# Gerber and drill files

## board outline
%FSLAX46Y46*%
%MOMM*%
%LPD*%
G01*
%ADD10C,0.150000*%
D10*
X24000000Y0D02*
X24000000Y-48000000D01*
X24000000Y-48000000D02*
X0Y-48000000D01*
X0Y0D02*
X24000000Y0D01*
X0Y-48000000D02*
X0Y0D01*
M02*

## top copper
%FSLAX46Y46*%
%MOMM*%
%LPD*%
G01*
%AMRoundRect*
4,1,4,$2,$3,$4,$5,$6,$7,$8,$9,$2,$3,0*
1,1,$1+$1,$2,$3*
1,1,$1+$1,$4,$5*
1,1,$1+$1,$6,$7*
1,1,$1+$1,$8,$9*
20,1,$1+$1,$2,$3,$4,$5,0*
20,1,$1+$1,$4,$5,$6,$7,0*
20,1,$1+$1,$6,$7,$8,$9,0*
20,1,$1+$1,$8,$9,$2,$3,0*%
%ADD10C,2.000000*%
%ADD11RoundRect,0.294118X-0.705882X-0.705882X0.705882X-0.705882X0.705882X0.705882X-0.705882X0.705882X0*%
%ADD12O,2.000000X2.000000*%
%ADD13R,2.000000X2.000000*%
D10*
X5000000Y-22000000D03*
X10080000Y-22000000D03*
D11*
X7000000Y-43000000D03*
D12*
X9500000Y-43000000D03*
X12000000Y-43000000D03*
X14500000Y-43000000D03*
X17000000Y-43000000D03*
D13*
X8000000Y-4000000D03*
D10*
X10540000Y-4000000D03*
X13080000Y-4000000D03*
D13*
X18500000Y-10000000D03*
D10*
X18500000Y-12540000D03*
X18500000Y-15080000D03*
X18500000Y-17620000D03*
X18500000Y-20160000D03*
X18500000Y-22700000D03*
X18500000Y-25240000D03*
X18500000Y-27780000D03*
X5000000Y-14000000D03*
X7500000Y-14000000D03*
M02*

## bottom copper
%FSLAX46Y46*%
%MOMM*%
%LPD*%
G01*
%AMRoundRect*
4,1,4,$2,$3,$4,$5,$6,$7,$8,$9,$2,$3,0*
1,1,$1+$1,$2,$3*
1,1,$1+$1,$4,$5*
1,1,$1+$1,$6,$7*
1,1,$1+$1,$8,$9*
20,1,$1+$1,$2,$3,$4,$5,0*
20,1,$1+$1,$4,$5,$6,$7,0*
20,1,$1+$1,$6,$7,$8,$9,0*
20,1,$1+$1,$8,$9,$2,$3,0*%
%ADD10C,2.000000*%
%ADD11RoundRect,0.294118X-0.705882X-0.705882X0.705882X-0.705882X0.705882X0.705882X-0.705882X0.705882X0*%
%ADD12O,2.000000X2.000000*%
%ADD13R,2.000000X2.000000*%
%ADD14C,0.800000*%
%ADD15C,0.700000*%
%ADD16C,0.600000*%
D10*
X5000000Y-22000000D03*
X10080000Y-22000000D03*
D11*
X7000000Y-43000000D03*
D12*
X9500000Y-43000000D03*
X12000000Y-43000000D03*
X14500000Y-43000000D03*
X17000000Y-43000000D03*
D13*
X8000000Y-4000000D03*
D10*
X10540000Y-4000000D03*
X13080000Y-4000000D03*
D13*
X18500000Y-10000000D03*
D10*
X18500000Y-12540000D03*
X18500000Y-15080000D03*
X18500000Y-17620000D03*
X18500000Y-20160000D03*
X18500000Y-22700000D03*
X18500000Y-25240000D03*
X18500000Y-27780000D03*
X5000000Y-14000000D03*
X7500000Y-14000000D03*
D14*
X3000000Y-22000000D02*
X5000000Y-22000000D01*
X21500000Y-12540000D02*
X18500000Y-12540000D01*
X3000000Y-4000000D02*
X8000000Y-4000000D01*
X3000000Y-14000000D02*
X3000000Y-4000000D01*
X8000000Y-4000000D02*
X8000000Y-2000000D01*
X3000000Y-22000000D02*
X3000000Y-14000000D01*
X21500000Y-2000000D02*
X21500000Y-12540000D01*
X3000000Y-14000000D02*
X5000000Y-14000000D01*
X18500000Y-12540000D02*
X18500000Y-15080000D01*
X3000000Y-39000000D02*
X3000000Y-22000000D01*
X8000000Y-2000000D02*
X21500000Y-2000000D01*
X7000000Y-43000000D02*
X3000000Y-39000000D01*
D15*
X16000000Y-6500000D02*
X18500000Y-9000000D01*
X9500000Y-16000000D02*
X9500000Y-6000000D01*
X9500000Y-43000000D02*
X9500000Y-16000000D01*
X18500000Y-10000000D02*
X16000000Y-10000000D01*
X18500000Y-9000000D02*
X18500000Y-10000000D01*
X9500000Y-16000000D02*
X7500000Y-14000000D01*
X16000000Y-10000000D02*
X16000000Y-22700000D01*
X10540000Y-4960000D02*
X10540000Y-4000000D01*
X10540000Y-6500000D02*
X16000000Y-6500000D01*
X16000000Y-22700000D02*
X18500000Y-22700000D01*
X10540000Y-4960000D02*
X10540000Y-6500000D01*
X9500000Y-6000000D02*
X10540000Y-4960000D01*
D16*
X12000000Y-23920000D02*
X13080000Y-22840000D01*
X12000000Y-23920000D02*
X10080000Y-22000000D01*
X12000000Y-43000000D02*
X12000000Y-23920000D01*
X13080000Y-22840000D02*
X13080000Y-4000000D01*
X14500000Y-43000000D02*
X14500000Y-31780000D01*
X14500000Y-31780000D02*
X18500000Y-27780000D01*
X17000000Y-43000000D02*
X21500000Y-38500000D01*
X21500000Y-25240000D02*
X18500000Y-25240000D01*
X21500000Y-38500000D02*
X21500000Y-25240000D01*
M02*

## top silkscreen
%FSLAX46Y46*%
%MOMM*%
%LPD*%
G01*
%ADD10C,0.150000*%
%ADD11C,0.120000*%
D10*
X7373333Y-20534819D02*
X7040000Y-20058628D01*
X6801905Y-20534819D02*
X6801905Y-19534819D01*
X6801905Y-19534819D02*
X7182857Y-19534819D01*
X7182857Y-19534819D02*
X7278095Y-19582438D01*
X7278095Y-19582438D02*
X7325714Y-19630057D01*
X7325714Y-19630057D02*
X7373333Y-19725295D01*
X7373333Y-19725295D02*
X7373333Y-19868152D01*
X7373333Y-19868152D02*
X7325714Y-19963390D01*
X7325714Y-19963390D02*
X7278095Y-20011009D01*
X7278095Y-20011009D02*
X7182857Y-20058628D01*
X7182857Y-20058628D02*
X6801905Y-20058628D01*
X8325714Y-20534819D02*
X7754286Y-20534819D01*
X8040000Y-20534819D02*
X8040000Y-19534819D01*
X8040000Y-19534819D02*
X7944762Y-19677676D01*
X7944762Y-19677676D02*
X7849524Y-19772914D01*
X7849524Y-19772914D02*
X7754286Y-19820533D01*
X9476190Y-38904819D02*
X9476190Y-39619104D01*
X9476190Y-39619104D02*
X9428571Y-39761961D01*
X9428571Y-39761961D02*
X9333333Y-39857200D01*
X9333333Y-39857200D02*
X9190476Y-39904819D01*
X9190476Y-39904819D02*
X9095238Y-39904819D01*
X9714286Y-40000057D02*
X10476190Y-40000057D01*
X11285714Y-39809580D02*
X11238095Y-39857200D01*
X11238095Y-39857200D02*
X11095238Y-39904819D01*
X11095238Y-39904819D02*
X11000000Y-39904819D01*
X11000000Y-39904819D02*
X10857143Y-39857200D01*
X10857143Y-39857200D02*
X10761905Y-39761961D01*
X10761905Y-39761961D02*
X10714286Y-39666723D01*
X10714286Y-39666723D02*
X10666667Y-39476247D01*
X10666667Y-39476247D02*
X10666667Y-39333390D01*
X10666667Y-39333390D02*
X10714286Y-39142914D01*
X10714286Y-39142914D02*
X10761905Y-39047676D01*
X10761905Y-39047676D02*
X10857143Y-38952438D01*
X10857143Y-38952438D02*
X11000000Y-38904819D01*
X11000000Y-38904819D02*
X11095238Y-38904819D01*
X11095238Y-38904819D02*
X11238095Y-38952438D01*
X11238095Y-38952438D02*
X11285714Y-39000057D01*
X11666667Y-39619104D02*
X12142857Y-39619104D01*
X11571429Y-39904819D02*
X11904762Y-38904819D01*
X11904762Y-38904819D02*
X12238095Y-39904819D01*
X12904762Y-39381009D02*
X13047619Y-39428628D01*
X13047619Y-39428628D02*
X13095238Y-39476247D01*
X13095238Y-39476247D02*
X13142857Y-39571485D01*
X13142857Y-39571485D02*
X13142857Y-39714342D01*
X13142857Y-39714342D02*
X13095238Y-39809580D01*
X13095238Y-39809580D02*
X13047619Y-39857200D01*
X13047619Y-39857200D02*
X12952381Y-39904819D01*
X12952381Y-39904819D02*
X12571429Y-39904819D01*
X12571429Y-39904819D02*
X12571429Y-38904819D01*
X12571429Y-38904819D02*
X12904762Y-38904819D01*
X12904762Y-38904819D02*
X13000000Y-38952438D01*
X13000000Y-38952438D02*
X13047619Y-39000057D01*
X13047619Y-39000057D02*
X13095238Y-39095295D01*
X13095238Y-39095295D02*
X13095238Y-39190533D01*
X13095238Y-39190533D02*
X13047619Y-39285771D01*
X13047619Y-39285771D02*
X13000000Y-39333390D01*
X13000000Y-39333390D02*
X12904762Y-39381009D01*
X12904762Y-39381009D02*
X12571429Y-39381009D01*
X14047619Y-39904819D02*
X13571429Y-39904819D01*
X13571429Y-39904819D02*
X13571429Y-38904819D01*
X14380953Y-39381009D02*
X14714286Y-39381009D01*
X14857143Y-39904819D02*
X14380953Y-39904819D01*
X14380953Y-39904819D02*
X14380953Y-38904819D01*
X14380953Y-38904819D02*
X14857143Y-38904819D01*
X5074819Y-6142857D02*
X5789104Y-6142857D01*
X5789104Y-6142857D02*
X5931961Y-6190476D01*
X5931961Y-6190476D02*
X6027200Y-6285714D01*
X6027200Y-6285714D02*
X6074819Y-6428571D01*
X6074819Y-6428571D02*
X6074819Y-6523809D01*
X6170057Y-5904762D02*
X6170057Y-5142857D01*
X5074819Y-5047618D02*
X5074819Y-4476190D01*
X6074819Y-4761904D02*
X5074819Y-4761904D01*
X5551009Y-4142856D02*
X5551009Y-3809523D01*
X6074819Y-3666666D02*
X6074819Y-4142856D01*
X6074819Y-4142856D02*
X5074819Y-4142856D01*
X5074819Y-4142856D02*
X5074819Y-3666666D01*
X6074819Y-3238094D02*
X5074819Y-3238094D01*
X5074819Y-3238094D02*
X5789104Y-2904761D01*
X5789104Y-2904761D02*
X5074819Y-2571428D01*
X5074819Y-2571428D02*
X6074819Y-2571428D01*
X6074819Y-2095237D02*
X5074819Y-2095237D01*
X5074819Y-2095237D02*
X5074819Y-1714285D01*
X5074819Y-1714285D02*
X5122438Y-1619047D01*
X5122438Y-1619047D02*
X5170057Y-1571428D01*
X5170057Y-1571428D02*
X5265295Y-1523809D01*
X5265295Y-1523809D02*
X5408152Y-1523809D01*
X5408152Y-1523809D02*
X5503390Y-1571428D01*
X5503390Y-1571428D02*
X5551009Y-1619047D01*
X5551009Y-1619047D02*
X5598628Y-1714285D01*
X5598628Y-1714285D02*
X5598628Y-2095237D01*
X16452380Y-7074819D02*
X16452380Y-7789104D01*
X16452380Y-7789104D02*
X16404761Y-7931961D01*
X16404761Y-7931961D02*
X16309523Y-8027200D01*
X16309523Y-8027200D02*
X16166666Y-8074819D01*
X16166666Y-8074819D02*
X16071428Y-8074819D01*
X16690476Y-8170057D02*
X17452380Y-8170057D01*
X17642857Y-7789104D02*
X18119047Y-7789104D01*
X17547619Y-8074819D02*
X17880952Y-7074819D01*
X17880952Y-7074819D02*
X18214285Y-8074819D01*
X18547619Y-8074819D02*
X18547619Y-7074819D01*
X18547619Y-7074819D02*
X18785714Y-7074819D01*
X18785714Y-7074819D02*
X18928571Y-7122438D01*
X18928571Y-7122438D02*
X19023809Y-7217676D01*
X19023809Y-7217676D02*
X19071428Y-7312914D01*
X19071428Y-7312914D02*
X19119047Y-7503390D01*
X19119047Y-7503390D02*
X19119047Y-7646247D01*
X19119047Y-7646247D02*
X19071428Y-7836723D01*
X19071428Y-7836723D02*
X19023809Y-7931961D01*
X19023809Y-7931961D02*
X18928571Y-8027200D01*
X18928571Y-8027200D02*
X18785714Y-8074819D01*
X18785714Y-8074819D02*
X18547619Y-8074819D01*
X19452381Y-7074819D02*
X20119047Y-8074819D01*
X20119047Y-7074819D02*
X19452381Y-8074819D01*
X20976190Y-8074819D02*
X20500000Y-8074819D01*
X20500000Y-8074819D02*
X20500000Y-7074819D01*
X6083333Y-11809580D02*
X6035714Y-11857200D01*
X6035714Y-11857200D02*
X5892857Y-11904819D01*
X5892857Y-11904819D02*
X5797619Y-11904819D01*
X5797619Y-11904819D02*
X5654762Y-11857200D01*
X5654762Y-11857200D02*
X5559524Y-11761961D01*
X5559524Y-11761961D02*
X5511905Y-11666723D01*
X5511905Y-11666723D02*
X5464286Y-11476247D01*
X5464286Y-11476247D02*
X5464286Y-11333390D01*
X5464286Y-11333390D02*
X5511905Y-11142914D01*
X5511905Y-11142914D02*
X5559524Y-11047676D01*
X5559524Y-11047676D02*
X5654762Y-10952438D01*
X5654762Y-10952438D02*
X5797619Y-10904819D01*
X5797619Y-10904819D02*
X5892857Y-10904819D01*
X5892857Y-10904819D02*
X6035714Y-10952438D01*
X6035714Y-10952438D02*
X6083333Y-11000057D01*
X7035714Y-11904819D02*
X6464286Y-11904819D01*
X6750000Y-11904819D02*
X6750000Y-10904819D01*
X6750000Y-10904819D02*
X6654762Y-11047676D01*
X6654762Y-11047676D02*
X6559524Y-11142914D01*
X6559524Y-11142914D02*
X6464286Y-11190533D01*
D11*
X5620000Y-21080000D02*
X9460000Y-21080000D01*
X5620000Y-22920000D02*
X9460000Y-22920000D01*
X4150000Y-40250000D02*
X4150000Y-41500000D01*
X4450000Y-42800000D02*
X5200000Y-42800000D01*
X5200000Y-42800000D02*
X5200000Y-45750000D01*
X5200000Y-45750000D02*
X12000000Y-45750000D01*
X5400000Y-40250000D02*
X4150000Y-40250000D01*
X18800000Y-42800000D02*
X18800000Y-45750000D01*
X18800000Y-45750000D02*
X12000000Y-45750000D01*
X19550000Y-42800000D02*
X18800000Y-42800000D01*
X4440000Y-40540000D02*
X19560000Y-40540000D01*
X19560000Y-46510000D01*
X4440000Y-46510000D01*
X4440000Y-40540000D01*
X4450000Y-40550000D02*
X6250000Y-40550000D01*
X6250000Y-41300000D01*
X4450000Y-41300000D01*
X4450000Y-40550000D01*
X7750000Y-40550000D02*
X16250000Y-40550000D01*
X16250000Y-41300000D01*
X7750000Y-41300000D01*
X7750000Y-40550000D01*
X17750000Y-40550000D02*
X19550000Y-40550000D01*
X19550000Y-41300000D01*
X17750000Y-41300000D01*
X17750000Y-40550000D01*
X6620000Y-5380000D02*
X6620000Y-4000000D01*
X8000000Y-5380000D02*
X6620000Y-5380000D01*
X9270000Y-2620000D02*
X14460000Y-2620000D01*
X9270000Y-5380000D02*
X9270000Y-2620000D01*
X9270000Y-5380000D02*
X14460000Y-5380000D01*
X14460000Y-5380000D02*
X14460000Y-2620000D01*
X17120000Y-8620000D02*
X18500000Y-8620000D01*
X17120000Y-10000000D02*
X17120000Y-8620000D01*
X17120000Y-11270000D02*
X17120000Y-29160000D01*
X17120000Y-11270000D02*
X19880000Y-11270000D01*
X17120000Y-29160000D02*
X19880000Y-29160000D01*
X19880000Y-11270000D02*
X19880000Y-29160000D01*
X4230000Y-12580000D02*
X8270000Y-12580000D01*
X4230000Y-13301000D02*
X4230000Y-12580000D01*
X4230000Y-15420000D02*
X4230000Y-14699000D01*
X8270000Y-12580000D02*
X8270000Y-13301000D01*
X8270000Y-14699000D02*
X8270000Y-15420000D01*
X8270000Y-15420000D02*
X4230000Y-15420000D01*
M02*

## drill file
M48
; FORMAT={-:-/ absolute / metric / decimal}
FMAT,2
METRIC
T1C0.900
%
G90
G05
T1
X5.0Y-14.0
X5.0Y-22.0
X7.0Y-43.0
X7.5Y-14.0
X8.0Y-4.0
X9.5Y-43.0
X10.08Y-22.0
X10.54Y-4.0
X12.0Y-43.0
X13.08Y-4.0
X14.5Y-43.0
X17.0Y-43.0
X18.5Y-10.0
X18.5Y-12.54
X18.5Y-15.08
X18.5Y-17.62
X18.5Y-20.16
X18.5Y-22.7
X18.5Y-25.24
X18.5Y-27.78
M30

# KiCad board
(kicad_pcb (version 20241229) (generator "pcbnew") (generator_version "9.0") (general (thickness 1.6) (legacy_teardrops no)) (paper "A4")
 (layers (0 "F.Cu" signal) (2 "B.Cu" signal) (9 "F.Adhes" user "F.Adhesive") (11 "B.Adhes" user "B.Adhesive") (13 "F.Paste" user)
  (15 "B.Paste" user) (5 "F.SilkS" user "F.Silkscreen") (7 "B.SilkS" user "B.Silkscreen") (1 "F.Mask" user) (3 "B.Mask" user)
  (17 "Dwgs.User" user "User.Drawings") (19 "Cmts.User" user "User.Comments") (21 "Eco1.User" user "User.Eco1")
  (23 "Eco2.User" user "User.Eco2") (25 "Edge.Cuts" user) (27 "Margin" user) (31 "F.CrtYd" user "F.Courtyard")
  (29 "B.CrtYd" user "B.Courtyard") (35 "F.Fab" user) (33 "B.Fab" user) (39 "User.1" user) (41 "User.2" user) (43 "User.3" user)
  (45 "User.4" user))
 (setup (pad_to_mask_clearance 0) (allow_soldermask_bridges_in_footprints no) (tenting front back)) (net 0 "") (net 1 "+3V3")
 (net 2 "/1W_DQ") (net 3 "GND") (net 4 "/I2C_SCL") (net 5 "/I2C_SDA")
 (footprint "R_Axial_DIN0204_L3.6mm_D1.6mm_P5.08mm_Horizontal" (layer "F.Cu") (at 5 22)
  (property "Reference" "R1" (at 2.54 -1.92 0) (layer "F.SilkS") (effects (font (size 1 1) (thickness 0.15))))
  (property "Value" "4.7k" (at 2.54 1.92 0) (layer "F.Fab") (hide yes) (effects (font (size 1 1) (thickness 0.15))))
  (fp_line (start 0.62 -0.92) (end 4.46 -0.92) (stroke (width 0.12) (type solid)) (layer "F.SilkS"))
  (fp_line (start 0.62 0.92) (end 4.46 0.92) (stroke (width 0.12) (type solid)) (layer "F.SilkS"))
  (pad "1" thru_hole circle (at 0 0) (size 2 2) (drill 0.9) (layers "*.Cu" "*.Mask") (remove_unused_layers no) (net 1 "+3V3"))
  (pad "2" thru_hole circle (at 5.08 0) (size 2 2) (drill 0.9) (layers "*.Cu" "*.Mask") (remove_unused_layers no) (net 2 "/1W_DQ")))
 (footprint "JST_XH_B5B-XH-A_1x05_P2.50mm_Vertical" (layer "F.Cu") (at 7 43)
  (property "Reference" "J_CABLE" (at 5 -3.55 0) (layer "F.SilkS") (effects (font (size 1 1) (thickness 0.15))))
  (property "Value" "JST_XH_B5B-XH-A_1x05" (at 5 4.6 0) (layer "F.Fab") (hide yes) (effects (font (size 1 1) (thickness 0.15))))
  (fp_line (start -2.85 -2.75) (end -2.85 -1.5) (stroke (width 0.12) (type solid)) (layer "F.SilkS"))
  (fp_line (start -2.55 -0.2) (end -1.8 -0.2) (stroke (width 0.12) (type solid)) (layer "F.SilkS"))
  (fp_line (start -1.8 -0.2) (end -1.8 2.75) (stroke (width 0.12) (type solid)) (layer "F.SilkS"))
  (fp_line (start -1.8 2.75) (end 5 2.75) (stroke (width 0.12) (type solid)) (layer "F.SilkS"))
  (fp_line (start -1.6 -2.75) (end -2.85 -2.75) (stroke (width 0.12) (type solid)) (layer "F.SilkS"))
  (fp_line (start 11.8 -0.2) (end 11.8 2.75) (stroke (width 0.12) (type solid)) (layer "F.SilkS"))
  (fp_line (start 11.8 2.75) (end 5 2.75) (stroke (width 0.12) (type solid)) (layer "F.SilkS"))
  (fp_line (start 12.55 -0.2) (end 11.8 -0.2) (stroke (width 0.12) (type solid)) (layer "F.SilkS"))
  (fp_rect (start -2.56 -2.46) (end 12.56 3.51) (stroke (width 0.12) (type solid)) (fill no) (layer "F.SilkS"))
  (fp_rect (start -2.55 -2.45) (end -0.75 -1.7) (stroke (width 0.12) (type solid)) (fill no) (layer "F.SilkS"))
  (fp_rect (start 0.75 -2.45) (end 9.25 -1.7) (stroke (width 0.12) (type solid)) (fill no) (layer "F.SilkS"))
  (fp_rect (start 10.75 -2.45) (end 12.55 -1.7) (stroke (width 0.12) (type solid)) (fill no) (layer "F.SilkS"))
  (pad "1" thru_hole roundrect (at 0 0) (size 2 2) (drill 0.9) (layers "*.Cu" "*.Mask") (remove_unused_layers no)
   (roundrect_rratio 0.147059) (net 1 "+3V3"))
  (pad "2" thru_hole oval (at 2.5 0) (size 2 2) (drill 0.9) (layers "*.Cu" "*.Mask") (remove_unused_layers no) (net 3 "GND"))
  (pad "3" thru_hole oval (at 5 0) (size 2 2) (drill 0.9) (layers "*.Cu" "*.Mask") (remove_unused_layers no) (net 2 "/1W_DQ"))
  (pad "4" thru_hole oval (at 7.5 0) (size 2 2) (drill 0.9) (layers "*.Cu" "*.Mask") (remove_unused_layers no) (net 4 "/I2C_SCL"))
  (pad "5" thru_hole oval (at 10 0) (size 2 2) (drill 0.9) (layers "*.Cu" "*.Mask") (remove_unused_layers no) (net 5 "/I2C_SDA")))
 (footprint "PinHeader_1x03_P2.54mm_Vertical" (layer "F.Cu") (at 8 4 90)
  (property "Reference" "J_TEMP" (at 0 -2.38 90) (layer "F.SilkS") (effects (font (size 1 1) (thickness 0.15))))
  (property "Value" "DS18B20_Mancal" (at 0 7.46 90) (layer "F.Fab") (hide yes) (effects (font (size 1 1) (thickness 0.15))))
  (fp_line (start -1.38 -1.38) (end 0 -1.38) (stroke (width 0.12) (type solid)) (layer "F.SilkS"))
  (fp_line (start -1.38 0) (end -1.38 -1.38) (stroke (width 0.12) (type solid)) (layer "F.SilkS"))
  (fp_line (start 1.38 1.27) (end 1.38 6.46) (stroke (width 0.12) (type solid)) (layer "F.SilkS"))
  (fp_line (start -1.38 1.27) (end 1.38 1.27) (stroke (width 0.12) (type solid)) (layer "F.SilkS"))
  (fp_line (start -1.38 1.27) (end -1.38 6.46) (stroke (width 0.12) (type solid)) (layer "F.SilkS"))
  (fp_line (start -1.38 6.46) (end 1.38 6.46) (stroke (width 0.12) (type solid)) (layer "F.SilkS"))
  (pad "1" thru_hole rect (at 0 0 90) (size 2 2) (drill 0.9) (layers "*.Cu" "*.Mask") (remove_unused_layers no) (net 1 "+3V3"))
  (pad "2" thru_hole circle (at 0 2.54 90) (size 2 2) (drill 0.9) (layers "*.Cu" "*.Mask") (remove_unused_layers no) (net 3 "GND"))
  (pad "3" thru_hole circle (at 0 5.08 90) (size 2 2) (drill 0.9) (layers "*.Cu" "*.Mask") (remove_unused_layers no) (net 2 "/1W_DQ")))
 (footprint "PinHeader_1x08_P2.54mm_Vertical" (layer "F.Cu") (at 18.5 10)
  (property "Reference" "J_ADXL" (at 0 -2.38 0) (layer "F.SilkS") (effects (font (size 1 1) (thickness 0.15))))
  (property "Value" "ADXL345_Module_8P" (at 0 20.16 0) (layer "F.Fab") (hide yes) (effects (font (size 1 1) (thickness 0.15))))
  (fp_line (start -1.38 -1.38) (end 0 -1.38) (stroke (width 0.12) (type solid)) (layer "F.SilkS"))
  (fp_line (start -1.38 0) (end -1.38 -1.38) (stroke (width 0.12) (type solid)) (layer "F.SilkS"))
  (fp_line (start -1.38 1.27) (end -1.38 19.16) (stroke (width 0.12) (type solid)) (layer "F.SilkS"))
  (fp_line (start -1.38 1.27) (end 1.38 1.27) (stroke (width 0.12) (type solid)) (layer "F.SilkS"))
  (fp_line (start -1.38 19.16) (end 1.38 19.16) (stroke (width 0.12) (type solid)) (layer "F.SilkS"))
  (fp_line (start 1.38 1.27) (end 1.38 19.16) (stroke (width 0.12) (type solid)) (layer "F.SilkS"))
  (pad "1" thru_hole rect (at 0 0) (size 2 2) (drill 0.9) (layers "*.Cu" "*.Mask") (remove_unused_layers no) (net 3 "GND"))
  (pad "2" thru_hole circle (at 0 2.54) (size 2 2) (drill 0.9) (layers "*.Cu" "*.Mask") (remove_unused_layers no) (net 1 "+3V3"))
  (pad "3" thru_hole circle (at 0 5.08) (size 2 2) (drill 0.9) (layers "*.Cu" "*.Mask") (remove_unused_layers no) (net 1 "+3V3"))
  (pad "4" thru_hole circle (at 0 7.62) (size 2 2) (drill 0.9) (layers "*.Cu" "*.Mask") (remove_unused_layers no))
  (pad "5" thru_hole circle (at 0 10.16) (size 2 2) (drill 0.9) (layers "*.Cu" "*.Mask") (remove_unused_layers no))
  (pad "6" thru_hole circle (at 0 12.7) (size 2 2) (drill 0.9) (layers "*.Cu" "*.Mask") (remove_unused_layers no) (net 3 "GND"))
  (pad "7" thru_hole circle (at 0 15.24) (size 2 2) (drill 0.9) (layers "*.Cu" "*.Mask") (remove_unused_layers no) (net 5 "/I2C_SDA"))
  (pad "8" thru_hole circle (at 0 17.78) (size 2 2) (drill 0.9) (layers "*.Cu" "*.Mask") (remove_unused_layers no) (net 4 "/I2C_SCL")))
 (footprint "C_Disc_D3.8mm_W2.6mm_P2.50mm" (layer "F.Cu") (at 5 14)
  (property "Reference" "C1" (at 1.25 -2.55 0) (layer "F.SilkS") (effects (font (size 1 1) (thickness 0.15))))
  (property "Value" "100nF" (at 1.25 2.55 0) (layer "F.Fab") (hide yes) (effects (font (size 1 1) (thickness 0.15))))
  (fp_line (start -0.77 -1.42) (end 3.27 -1.42) (stroke (width 0.12) (type solid)) (layer "F.SilkS"))
  (fp_line (start -0.77 -0.699) (end -0.77 -1.42) (stroke (width 0.12) (type solid)) (layer "F.SilkS"))
  (fp_line (start -0.77 1.42) (end -0.77 0.699) (stroke (width 0.12) (type solid)) (layer "F.SilkS"))
  (fp_line (start 3.27 -1.42) (end 3.27 -0.699) (stroke (width 0.12) (type solid)) (layer "F.SilkS"))
  (fp_line (start 3.27 0.699) (end 3.27 1.42) (stroke (width 0.12) (type solid)) (layer "F.SilkS"))
  (fp_line (start 3.27 1.42) (end -0.77 1.42) (stroke (width 0.12) (type solid)) (layer "F.SilkS"))
  (pad "1" thru_hole circle (at 0 0) (size 2 2) (drill 0.9) (layers "*.Cu" "*.Mask") (remove_unused_layers no) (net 1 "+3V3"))
  (pad "2" thru_hole circle (at 2.5 0) (size 2 2) (drill 0.9) (layers "*.Cu" "*.Mask") (remove_unused_layers no) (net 3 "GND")))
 (gr_line (start 24 0) (end 24 48) (stroke (width 0.15) (type default)) (layer "Edge.Cuts"))
 (gr_line (start 24 48) (end 0 48) (stroke (width 0.15) (type default)) (layer "Edge.Cuts"))
 (gr_line (start 0 0) (end 24 0) (stroke (width 0.15) (type default)) (layer "Edge.Cuts"))
 (gr_line (start 0 48) (end 0 0) (stroke (width 0.15) (type default)) (layer "Edge.Cuts"))
 (segment (start 3 22) (end 5 22) (width 0.8) (layer "B.Cu") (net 1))
 (segment (start 21.5 12.54) (end 18.5 12.54) (width 0.8) (layer "B.Cu") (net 1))
 (segment (start 3 4) (end 8 4) (width 0.8) (layer "B.Cu") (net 1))
 (segment (start 3 14) (end 3 4) (width 0.8) (layer "B.Cu") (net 1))
 (segment (start 8 4) (end 8 2) (width 0.8) (layer "B.Cu") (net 1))
 (segment (start 3 22) (end 3 14) (width 0.8) (layer "B.Cu") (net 1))
 (segment (start 21.5 2) (end 21.5 12.54) (width 0.8) (layer "B.Cu") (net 1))
 (segment (start 3 14) (end 5 14) (width 0.8) (layer "B.Cu") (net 1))
 (segment (start 18.5 12.54) (end 18.5 15.08) (width 0.8) (layer "B.Cu") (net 1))
 (segment (start 3 39) (end 3 22) (width 0.8) (layer "B.Cu") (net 1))
 (segment (start 8 2) (end 21.5 2) (width 0.8) (layer "B.Cu") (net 1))
 (segment (start 7 43) (end 3 39) (width 0.8) (layer "B.Cu") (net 1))
 (segment (start 16 6.5) (end 18.5 9) (width 0.7) (layer "B.Cu") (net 3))
 (segment (start 9.5 16) (end 9.5 6) (width 0.7) (layer "B.Cu") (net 3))
 (segment (start 9.5 43) (end 9.5 16) (width 0.7) (layer "B.Cu") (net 3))
 (segment (start 18.5 10) (end 16 10) (width 0.7) (layer "B.Cu") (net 3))
 (segment (start 18.5 9) (end 18.5 10) (width 0.7) (layer "B.Cu") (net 3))
 (segment (start 9.5 16) (end 7.5 14) (width 0.7) (layer "B.Cu") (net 3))
 (segment (start 16 10) (end 16 22.7) (width 0.7) (layer "B.Cu") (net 3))
 (segment (start 10.54 4.96) (end 10.54 4) (width 0.7) (layer "B.Cu") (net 3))
 (segment (start 10.54 6.5) (end 16 6.5) (width 0.7) (layer "B.Cu") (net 3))
 (segment (start 16 22.7) (end 18.5 22.7) (width 0.7) (layer "B.Cu") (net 3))
 (segment (start 10.54 4.96) (end 10.54 6.5) (width 0.7) (layer "B.Cu") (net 3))
 (segment (start 9.5 6) (end 10.54 4.96) (width 0.7) (layer "B.Cu") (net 3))
 (segment (start 12 23.92) (end 13.08 22.84) (width 0.6) (layer "B.Cu") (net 2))
 (segment (start 12 23.92) (end 10.08 22) (width 0.6) (layer "B.Cu") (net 2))
 (segment (start 12 43) (end 12 23.92) (width 0.6) (layer "B.Cu") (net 2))
 (segment (start 13.08 22.84) (end 13.08 4) (width 0.6) (layer "B.Cu") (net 2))
 (segment (start 14.5 43) (end 14.5 31.78) (width 0.6) (layer "B.Cu") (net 4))
 (segment (start 14.5 31.78) (end 18.5 27.78) (width 0.6) (layer "B.Cu") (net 4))
 (segment (start 17 43) (end 21.5 38.5) (width 0.6) (layer "B.Cu") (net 5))
 (segment (start 21.5 25.24) (end 18.5 25.24) (width 0.6) (layer "B.Cu") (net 5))
 (segment (start 21.5 38.5) (end 21.5 25.24) (width 0.6) (layer "B.Cu") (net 5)))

